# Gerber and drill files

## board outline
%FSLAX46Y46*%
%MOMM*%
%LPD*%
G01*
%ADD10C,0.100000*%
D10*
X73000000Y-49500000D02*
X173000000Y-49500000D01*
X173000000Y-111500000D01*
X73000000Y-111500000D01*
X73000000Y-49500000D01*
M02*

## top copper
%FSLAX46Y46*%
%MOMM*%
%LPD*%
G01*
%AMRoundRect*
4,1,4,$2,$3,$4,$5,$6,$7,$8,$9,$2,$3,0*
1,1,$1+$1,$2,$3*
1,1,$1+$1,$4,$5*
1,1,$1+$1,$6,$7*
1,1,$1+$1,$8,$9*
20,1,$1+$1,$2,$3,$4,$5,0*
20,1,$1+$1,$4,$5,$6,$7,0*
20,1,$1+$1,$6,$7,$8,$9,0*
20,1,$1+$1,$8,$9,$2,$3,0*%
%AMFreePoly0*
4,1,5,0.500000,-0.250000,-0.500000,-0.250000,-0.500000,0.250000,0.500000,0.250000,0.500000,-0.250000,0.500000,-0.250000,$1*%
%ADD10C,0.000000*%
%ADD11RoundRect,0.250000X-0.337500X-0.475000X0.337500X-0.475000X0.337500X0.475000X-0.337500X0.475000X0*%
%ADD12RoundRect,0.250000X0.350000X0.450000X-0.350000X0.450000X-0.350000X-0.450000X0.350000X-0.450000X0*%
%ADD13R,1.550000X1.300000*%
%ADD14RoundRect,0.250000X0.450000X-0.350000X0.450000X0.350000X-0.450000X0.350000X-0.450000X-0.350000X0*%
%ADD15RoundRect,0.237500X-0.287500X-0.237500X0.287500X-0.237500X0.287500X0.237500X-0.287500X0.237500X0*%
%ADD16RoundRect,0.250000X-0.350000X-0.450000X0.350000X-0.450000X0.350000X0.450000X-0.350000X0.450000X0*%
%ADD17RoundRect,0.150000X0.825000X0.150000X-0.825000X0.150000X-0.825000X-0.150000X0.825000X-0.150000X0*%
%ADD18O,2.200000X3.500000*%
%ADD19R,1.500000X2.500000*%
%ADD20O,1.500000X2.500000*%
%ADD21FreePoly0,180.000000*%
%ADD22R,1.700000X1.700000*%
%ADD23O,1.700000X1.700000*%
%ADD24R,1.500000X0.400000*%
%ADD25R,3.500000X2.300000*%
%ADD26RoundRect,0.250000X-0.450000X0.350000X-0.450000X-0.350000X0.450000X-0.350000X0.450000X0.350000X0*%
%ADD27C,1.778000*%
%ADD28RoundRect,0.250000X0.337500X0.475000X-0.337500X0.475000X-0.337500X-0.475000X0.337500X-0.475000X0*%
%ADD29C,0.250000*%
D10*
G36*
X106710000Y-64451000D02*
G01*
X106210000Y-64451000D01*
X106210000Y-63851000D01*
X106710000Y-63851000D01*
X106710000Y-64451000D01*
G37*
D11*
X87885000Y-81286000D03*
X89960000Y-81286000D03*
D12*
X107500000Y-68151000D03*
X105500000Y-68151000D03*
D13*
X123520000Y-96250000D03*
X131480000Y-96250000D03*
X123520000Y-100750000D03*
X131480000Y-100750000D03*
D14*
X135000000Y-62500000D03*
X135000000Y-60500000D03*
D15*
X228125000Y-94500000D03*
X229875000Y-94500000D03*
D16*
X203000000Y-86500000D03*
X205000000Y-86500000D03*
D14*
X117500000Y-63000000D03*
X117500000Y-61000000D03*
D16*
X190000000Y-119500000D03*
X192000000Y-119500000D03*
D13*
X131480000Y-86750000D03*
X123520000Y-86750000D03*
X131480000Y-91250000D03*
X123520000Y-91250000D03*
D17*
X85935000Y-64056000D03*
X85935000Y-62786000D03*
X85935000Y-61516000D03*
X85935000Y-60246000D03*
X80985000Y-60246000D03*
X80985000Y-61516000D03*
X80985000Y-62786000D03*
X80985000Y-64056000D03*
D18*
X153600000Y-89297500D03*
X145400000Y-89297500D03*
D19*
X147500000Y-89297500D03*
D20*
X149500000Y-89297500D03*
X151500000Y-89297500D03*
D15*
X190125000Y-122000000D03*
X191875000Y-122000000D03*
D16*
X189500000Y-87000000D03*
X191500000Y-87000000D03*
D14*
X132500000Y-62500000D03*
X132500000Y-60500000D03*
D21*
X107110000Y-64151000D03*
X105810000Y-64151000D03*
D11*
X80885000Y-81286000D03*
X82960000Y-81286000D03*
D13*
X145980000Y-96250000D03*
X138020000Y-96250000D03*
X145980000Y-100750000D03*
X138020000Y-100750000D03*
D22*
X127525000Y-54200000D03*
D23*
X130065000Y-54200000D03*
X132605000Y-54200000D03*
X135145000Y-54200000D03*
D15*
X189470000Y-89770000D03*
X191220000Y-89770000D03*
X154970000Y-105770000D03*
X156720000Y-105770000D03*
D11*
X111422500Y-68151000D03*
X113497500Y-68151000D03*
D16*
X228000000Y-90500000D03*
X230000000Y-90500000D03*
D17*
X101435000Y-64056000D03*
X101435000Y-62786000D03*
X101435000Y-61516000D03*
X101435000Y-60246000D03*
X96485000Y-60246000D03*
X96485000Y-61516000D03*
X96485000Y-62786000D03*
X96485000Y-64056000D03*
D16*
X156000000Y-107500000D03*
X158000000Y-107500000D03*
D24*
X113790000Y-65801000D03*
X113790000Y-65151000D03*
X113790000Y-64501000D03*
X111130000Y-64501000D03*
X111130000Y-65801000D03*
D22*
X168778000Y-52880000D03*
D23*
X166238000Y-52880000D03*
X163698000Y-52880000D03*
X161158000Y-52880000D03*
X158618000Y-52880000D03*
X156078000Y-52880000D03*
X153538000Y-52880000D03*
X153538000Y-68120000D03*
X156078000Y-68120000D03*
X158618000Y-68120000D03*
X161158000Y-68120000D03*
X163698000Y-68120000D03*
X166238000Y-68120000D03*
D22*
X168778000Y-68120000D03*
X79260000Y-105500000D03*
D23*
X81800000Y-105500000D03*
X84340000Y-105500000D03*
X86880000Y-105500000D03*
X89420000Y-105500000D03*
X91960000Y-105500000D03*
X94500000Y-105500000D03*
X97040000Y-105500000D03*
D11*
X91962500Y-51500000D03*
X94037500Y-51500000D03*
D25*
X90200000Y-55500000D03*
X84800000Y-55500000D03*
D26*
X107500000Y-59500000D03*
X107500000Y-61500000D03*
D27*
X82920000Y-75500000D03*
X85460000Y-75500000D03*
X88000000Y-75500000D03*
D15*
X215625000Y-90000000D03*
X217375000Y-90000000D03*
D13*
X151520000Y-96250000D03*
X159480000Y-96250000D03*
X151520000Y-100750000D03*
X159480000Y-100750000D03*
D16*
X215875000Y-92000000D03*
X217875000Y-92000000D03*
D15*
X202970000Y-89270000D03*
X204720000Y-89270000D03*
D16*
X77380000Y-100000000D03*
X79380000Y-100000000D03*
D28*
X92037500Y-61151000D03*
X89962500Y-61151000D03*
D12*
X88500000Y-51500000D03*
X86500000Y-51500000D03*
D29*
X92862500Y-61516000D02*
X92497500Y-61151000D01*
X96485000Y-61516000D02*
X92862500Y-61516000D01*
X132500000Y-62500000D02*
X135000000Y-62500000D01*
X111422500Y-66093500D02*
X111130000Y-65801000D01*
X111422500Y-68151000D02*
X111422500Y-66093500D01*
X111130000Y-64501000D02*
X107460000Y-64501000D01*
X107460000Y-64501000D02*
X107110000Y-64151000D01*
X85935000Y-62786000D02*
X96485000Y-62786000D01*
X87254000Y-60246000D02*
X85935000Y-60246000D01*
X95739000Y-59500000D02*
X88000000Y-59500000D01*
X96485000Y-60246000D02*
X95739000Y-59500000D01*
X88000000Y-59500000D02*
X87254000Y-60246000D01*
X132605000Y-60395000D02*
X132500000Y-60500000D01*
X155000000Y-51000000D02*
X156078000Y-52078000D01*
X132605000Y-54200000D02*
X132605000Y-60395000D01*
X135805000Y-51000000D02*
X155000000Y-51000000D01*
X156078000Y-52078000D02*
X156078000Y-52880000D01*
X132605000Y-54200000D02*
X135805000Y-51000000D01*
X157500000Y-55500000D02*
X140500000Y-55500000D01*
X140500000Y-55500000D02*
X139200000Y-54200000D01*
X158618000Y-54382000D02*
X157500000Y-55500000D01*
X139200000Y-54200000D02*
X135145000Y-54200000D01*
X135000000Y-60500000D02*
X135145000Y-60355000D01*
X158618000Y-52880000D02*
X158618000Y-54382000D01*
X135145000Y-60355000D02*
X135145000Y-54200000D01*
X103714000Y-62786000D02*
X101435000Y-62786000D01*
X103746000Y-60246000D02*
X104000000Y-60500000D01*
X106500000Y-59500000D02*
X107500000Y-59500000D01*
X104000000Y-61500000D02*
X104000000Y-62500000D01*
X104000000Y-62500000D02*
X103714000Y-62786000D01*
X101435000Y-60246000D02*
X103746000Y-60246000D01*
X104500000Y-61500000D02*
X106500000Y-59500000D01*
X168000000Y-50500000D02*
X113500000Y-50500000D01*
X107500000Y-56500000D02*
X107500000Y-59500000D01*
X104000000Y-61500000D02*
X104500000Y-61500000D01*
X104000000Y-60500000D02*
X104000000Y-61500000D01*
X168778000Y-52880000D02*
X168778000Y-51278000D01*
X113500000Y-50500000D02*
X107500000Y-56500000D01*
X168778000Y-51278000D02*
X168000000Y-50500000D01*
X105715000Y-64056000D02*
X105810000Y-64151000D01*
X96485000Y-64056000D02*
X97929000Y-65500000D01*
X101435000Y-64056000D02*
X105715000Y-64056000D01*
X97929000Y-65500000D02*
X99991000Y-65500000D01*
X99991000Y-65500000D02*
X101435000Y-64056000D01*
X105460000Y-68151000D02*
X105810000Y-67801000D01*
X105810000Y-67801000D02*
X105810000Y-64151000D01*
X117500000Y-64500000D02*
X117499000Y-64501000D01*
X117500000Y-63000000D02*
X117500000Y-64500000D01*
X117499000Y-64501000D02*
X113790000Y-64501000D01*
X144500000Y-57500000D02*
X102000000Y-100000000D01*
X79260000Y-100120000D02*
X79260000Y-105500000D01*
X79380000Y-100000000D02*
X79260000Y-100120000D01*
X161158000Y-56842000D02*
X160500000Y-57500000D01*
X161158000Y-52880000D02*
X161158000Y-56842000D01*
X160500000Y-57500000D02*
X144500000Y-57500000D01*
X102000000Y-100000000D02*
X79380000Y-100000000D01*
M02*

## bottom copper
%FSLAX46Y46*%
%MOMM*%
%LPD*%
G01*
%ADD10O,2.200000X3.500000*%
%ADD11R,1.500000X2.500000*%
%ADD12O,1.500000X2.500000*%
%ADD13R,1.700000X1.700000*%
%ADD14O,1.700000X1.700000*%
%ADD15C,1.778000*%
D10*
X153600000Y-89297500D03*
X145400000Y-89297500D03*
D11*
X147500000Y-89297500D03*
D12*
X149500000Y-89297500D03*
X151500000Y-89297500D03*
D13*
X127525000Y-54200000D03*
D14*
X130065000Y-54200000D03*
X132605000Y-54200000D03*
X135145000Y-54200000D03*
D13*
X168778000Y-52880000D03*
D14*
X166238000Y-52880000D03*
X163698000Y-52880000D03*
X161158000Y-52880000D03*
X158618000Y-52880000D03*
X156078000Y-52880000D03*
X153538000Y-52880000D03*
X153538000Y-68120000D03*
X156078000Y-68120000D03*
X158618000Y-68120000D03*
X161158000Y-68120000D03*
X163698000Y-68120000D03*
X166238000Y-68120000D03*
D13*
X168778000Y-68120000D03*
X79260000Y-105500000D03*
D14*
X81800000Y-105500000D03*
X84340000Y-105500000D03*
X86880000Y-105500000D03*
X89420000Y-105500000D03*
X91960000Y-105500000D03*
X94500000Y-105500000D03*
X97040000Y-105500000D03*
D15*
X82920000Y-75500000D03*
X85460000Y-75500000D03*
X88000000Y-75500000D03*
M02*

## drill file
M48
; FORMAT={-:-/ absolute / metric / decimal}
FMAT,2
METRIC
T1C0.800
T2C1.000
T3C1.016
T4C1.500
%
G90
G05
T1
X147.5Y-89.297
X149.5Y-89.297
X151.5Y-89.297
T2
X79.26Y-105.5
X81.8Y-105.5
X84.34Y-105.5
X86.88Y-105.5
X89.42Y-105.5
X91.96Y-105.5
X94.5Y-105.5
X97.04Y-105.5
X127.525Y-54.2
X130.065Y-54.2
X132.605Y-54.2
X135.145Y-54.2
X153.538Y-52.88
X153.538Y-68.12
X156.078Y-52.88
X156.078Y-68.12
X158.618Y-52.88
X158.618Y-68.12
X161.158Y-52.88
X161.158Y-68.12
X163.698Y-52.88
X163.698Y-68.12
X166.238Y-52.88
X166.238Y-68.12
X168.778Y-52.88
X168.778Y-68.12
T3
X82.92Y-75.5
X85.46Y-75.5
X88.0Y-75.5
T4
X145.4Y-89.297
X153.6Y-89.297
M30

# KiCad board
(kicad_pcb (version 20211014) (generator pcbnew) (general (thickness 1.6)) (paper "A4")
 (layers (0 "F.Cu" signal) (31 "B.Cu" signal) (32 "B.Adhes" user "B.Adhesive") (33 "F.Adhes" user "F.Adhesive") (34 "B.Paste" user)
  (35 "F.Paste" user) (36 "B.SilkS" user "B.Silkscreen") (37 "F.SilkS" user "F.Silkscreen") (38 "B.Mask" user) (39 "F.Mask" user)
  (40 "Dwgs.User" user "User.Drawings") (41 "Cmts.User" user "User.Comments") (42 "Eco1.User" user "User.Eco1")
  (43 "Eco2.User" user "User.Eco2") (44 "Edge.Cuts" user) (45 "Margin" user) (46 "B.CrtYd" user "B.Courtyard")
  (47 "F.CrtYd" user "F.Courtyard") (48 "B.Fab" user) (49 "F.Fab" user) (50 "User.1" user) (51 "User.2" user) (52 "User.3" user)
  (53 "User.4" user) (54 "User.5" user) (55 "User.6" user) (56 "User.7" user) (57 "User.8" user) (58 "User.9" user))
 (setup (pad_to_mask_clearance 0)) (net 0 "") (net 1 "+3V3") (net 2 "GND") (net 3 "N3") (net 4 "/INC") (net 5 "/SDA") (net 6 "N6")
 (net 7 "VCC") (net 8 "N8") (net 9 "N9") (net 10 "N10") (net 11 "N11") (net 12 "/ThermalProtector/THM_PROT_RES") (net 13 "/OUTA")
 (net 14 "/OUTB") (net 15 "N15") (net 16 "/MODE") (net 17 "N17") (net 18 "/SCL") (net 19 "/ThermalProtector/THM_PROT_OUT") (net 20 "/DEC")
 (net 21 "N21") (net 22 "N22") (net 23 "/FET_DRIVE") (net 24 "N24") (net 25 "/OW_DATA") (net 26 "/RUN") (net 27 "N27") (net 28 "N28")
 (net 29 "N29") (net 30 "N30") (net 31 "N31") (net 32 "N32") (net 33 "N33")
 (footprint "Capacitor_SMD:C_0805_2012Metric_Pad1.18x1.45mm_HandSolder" (layer "F.Cu") (at 88.9225 81.286)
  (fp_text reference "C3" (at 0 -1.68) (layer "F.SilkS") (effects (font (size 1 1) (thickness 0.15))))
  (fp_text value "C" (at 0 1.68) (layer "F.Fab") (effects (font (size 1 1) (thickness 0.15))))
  (pad "1" smd roundrect (at -1.0375 0) (size 1.175 1.45) (layers "F.Cu" "F.Paste" "F.Mask") (roundrect_rratio 0.212766) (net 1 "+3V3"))
  (pad "2" smd roundrect (at 1.0375 0) (size 1.175 1.45) (layers "F.Cu" "F.Paste" "F.Mask") (roundrect_rratio 0.212766) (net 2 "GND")))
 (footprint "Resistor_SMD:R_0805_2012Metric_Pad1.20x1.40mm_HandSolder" (layer "F.Cu") (at 106.5 68.151 180)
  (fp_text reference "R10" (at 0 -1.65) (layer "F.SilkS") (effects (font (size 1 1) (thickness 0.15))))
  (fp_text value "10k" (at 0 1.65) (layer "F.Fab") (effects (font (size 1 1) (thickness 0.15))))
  (pad "1" smd roundrect (at -1 0 180) (size 1.2 1.4) (layers "F.Cu" "F.Paste" "F.Mask") (roundrect_rratio 0.208333) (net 1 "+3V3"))
  (pad "2" smd roundrect (at 1 0 180) (size 1.2 1.4) (layers "F.Cu" "F.Paste" "F.Mask") (roundrect_rratio 0.208333) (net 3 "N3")))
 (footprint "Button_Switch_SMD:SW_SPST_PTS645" (layer "F.Cu") (at 127.5 98.5)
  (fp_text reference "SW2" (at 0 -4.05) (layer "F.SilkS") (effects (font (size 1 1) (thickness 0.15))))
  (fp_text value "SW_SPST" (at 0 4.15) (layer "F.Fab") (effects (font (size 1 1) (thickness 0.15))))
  (pad "1" smd rect (at -3.98 -2.25) (size 1.55 1.3) (layers "F.Cu" "F.Paste" "F.Mask") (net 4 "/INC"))
  (pad "1" smd rect (at 3.98 -2.25) (size 1.55 1.3) (layers "F.Cu" "F.Paste" "F.Mask") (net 4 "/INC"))
  (pad "2" smd rect (at -3.98 2.25) (size 1.55 1.3) (layers "F.Cu" "F.Paste" "F.Mask") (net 2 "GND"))
  (pad "2" smd rect (at 3.98 2.25) (size 1.55 1.3) (layers "F.Cu" "F.Paste" "F.Mask") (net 2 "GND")))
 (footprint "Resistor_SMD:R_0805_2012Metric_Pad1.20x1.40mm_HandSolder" (layer "F.Cu") (at 135 61.5 90)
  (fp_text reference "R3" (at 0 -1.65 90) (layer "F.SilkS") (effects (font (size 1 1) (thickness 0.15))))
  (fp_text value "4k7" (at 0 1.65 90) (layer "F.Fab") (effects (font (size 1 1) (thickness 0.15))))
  (pad "1" smd roundrect (at -1 0 90) (size 1.2 1.4) (layers "F.Cu" "F.Paste" "F.Mask") (roundrect_rratio 0.208333) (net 1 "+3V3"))
  (pad "2" smd roundrect (at 1 0 90) (size 1.2 1.4) (layers "F.Cu" "F.Paste" "F.Mask") (roundrect_rratio 0.208333) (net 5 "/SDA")))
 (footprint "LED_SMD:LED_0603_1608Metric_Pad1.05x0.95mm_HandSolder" (layer "F.Cu") (at 229 94.5)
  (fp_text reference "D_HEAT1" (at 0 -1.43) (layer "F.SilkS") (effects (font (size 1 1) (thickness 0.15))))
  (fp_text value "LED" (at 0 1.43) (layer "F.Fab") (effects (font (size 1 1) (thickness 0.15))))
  (pad "1" smd roundrect (at -0.875 0) (size 1.05 0.95) (layers "F.Cu" "F.Paste" "F.Mask") (roundrect_rratio 0.25) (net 2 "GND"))
  (pad "2" smd roundrect (at 0.875 0) (size 1.05 0.95) (layers "F.Cu" "F.Paste" "F.Mask") (roundrect_rratio 0.25) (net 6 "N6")))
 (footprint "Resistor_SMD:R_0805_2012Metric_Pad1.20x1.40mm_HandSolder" (layer "F.Cu") (at 204 86.5)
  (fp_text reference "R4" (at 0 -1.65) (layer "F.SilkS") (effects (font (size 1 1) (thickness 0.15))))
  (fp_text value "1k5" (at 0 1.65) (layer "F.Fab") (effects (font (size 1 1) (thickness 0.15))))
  (pad "1" smd roundrect (at -1 0) (size 1.2 1.4) (layers "F.Cu" "F.Paste" "F.Mask") (roundrect_rratio 0.208333) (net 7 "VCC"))
  (pad "2" smd roundrect (at 1 0) (size 1.2 1.4) (layers "F.Cu" "F.Paste" "F.Mask") (roundrect_rratio 0.208333) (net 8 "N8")))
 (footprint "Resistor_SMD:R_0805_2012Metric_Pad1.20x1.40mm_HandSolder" (layer "F.Cu") (at 117.5 62 90)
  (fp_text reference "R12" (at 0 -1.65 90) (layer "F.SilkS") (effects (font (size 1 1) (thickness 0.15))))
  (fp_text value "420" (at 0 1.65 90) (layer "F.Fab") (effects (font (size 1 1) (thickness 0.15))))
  (pad "1" smd roundrect (at -1 0 90) (size 1.2 1.4) (layers "F.Cu" "F.Paste" "F.Mask") (roundrect_rratio 0.208333) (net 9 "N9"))
  (pad "2" smd roundrect (at 1 0 90) (size 1.2 1.4) (layers "F.Cu" "F.Paste" "F.Mask") (roundrect_rratio 0.208333) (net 2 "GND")))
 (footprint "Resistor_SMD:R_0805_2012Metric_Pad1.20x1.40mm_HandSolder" (layer "F.Cu") (at 191 119.5)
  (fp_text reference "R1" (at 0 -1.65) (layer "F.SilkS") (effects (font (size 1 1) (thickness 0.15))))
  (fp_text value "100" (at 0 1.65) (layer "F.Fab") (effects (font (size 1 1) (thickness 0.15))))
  (pad "1" smd roundrect (at -1 0) (size 1.2 1.4) (layers "F.Cu" "F.Paste" "F.Mask") (roundrect_rratio 0.208333) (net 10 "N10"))
  (pad "2" smd roundrect (at 1 0) (size 1.2 1.4) (layers "F.Cu" "F.Paste" "F.Mask") (roundrect_rratio 0.208333) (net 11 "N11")))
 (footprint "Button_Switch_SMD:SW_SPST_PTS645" (layer "F.Cu") (at 127.5 89)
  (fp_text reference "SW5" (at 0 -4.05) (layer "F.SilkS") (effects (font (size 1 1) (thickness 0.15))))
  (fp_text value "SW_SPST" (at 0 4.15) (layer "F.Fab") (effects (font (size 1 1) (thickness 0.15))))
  (pad "1" smd rect (at 3.98 -2.25) (size 1.55 1.3) (layers "F.Cu" "F.Paste" "F.Mask") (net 2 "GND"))
  (pad "1" smd rect (at -3.98 -2.25) (size 1.55 1.3) (layers "F.Cu" "F.Paste" "F.Mask") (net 2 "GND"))
  (pad "2" smd rect (at 3.98 2.25) (size 1.55 1.3) (layers "F.Cu" "F.Paste" "F.Mask") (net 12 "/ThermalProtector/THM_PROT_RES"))
  (pad "2" smd rect (at -3.98 2.25) (size 1.55 1.3) (layers "F.Cu" "F.Paste" "F.Mask") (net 12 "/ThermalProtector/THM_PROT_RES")))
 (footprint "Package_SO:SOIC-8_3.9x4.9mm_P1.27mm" (layer "F.Cu") (at 83.46 62.151 180)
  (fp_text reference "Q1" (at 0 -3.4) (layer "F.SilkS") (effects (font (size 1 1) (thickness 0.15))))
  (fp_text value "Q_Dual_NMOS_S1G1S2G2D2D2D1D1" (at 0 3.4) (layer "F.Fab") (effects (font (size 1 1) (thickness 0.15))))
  (pad "1" smd roundrect (at -2.475 -1.905 180) (size 1.95 0.6) (layers "F.Cu" "F.Paste" "F.Mask") (roundrect_rratio 0.25) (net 2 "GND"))
  (pad "2" smd roundrect (at -2.475 -0.635 180) (size 1.95 0.6) (layers "F.Cu" "F.Paste" "F.Mask") (roundrect_rratio 0.25) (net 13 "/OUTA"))
  (pad "3" smd roundrect (at -2.475 0.635 180) (size 1.95 0.6) (layers "F.Cu" "F.Paste" "F.Mask") (roundrect_rratio 0.25) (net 2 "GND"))
  (pad "4" smd roundrect (at -2.475 1.905 180) (size 1.95 0.6) (layers "F.Cu" "F.Paste" "F.Mask") (roundrect_rratio 0.25) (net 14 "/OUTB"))
  (pad "5" smd roundrect (at 2.475 1.905 180) (size 1.95 0.6) (layers "F.Cu" "F.Paste" "F.Mask") (roundrect_rratio 0.25) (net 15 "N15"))
  (pad "6" smd roundrect (at 2.475 0.635 180) (size 1.95 0.6) (layers "F.Cu" "F.Paste" "F.Mask") (roundrect_rratio 0.25) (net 15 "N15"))
  (pad "7" smd roundrect (at 2.475 -0.635 180) (size 1.95 0.6) (layers "F.Cu" "F.Paste" "F.Mask") (roundrect_rratio 0.25) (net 15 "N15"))
  (pad "8" smd roundrect (at 2.475 -1.905 180) (size 1.95 0.6) (layers "F.Cu" "F.Paste" "F.Mask") (roundrect_rratio 0.25) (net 15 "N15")))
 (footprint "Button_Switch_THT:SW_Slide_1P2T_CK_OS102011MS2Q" (layer "F.Cu") (at 147.5 89.2975)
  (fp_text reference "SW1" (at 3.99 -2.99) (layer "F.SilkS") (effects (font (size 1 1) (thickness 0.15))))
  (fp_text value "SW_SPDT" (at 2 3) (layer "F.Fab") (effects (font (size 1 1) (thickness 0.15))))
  (pad "" thru_hole oval (at 6.1 0) (size 2.2 3.5) (drill 1.5) (layers *.Cu *.Mask))
  (pad "" thru_hole oval (at -2.1 0) (size 2.2 3.5) (drill 1.5) (layers *.Cu *.Mask))
  (pad "1" thru_hole rect (at 0 0) (size 1.5 2.5) (drill 0.8) (layers *.Cu *.Mask) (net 1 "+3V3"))
  (pad "2" thru_hole oval (at 2 0) (size 1.5 2.5) (drill 0.8) (layers *.Cu *.Mask) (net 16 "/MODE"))
  (pad "3" thru_hole oval (at 4 0) (size 1.5 2.5) (drill 0.8) (layers *.Cu *.Mask) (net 2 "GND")))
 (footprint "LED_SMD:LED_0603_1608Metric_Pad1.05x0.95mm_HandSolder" (layer "F.Cu") (at 191 122)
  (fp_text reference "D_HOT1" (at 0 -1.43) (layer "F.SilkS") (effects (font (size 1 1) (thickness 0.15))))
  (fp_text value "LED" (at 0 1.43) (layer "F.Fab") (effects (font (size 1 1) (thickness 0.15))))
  (pad "1" smd roundrect (at -0.875 0) (size 1.05 0.95) (layers "F.Cu" "F.Paste" "F.Mask") (roundrect_rratio 0.25) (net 2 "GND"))
  (pad "2" smd roundrect (at 0.875 0) (size 1.05 0.95) (layers "F.Cu" "F.Paste" "F.Mask") (roundrect_rratio 0.25) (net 11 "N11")))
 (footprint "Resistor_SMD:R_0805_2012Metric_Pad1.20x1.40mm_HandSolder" (layer "F.Cu") (at 190.5 87)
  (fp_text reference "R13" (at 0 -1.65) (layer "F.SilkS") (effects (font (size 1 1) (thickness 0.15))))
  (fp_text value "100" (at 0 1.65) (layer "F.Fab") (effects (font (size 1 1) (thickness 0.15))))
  (pad "1" smd roundrect (at -1 0) (size 1.2 1.4) (layers "F.Cu" "F.Paste" "F.Mask") (roundrect_rratio 0.208333) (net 1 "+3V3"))
  (pad "2" smd roundrect (at 1 0) (size 1.2 1.4) (layers "F.Cu" "F.Paste" "F.Mask") (roundrect_rratio 0.208333) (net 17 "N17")))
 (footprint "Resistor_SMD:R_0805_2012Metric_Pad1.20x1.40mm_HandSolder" (layer "F.Cu") (at 132.5 61.5 90)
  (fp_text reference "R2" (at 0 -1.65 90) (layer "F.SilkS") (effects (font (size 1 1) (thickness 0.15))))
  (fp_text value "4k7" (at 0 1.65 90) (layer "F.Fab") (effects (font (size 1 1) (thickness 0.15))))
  (pad "1" smd roundrect (at -1 0 90) (size 1.2 1.4) (layers "F.Cu" "F.Paste" "F.Mask") (roundrect_rratio 0.208333) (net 1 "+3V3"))
  (pad "2" smd roundrect (at 1 0 90) (size 1.2 1.4) (layers "F.Cu" "F.Paste" "F.Mask") (roundrect_rratio 0.208333) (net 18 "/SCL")))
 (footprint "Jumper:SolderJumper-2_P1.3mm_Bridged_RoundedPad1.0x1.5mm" (layer "F.Cu") (at 106.46 64.151 180)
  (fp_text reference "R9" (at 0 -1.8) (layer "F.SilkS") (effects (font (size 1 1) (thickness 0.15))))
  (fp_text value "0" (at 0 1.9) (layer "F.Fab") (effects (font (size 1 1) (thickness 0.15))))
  (fp_poly (pts (xy 0.25 -0.3) (xy -0.25 -0.3) (xy -0.25 0.3) (xy 0.25 0.3)) (layer "F.Cu") (width 0) (fill solid))
  (pad "1" smd custom (at -0.65 0 180) (size 1 0.5) (layers "F.Cu" "F.Mask") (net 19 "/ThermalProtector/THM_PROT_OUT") (zone_connect 2)
   (options (clearance outline) (anchor rect)) (primitives))
  (pad "2" smd custom (at 0.65 0 180) (size 1 0.5) (layers "F.Cu" "F.Mask") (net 3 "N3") (zone_connect 2)
   (options (clearance outline) (anchor rect)) (primitives)))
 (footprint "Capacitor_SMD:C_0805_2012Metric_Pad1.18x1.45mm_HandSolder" (layer "F.Cu") (at 81.9225 81.286)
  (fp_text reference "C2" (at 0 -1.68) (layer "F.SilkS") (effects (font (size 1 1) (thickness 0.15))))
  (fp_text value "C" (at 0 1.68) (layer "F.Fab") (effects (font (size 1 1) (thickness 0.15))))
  (pad "1" smd roundrect (at -1.0375 0) (size 1.175 1.45) (layers "F.Cu" "F.Paste" "F.Mask") (roundrect_rratio 0.212766) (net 7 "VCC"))
  (pad "2" smd roundrect (at 1.0375 0) (size 1.175 1.45) (layers "F.Cu" "F.Paste" "F.Mask") (roundrect_rratio 0.212766) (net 2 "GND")))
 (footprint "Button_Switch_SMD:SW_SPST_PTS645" (layer "F.Cu") (at 142 98.5)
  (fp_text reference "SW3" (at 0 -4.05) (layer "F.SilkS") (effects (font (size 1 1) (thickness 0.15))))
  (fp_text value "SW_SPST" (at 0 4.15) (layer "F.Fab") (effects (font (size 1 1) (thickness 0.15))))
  (pad "1" smd rect (at 3.98 -2.25) (size 1.55 1.3) (layers "F.Cu" "F.Paste" "F.Mask") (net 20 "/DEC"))
  (pad "1" smd rect (at -3.98 -2.25) (size 1.55 1.3) (layers "F.Cu" "F.Paste" "F.Mask") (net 20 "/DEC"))
  (pad "2" smd rect (at 3.98 2.25) (size 1.55 1.3) (layers "F.Cu" "F.Paste" "F.Mask") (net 2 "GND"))
  (pad "2" smd rect (at -3.98 2.25) (size 1.55 1.3) (layers "F.Cu" "F.Paste" "F.Mask") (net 2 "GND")))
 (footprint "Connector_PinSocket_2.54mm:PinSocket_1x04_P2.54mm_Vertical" (layer "F.Cu") (at 127.525 54.2 90)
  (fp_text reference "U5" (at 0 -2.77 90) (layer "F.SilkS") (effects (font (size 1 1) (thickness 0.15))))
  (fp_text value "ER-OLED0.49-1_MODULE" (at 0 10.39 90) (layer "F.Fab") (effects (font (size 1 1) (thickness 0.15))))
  (pad "1" thru_hole rect (at 0 0 90) (size 1.7 1.7) (drill 1) (layers *.Cu *.Mask) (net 2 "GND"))
  (pad "2" thru_hole oval (at 0 2.54 90) (size 1.7 1.7) (drill 1) (layers *.Cu *.Mask) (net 1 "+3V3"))
  (pad "3" thru_hole oval (at 0 5.08 90) (size 1.7 1.7) (drill 1) (layers *.Cu *.Mask) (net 18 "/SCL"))
  (pad "4" thru_hole oval (at 0 7.62 90) (size 1.7 1.7) (drill 1) (layers *.Cu *.Mask) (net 5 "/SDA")))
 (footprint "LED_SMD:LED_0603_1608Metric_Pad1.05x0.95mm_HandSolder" (layer "F.Cu") (at 190.345 89.77)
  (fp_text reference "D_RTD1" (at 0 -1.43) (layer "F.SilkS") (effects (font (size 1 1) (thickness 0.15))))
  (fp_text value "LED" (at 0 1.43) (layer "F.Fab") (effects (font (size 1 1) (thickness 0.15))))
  (pad "1" smd roundrect (at -0.875 0) (size 1.05 0.95) (layers "F.Cu" "F.Paste" "F.Mask") (roundrect_rratio 0.25)
   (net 19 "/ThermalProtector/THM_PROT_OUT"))
  (pad "2" smd roundrect (at 0.875 0) (size 1.05 0.95) (layers "F.Cu" "F.Paste" "F.Mask") (roundrect_rratio 0.25) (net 17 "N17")))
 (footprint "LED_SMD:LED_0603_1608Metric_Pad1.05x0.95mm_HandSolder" (layer "F.Cu") (at 155.845 105.77)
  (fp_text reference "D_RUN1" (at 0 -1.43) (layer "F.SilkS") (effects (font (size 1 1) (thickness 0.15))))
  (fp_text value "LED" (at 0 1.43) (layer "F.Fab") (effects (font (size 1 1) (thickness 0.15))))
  (pad "1" smd roundrect (at -0.875 0) (size 1.05 0.95) (layers "F.Cu" "F.Paste" "F.Mask") (roundrect_rratio 0.25) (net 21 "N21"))
  (pad "2" smd roundrect (at 0.875 0) (size 1.05 0.95) (layers "F.Cu" "F.Paste" "F.Mask") (roundrect_rratio 0.25) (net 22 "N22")))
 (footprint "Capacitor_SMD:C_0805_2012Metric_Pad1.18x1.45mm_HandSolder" (layer "F.Cu") (at 112.46 68.151)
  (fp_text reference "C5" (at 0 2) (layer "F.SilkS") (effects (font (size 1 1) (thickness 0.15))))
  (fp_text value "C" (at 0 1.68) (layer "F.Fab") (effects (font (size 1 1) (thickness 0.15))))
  (pad "1" smd roundrect (at -1.0375 0) (size 1.175 1.45) (layers "F.Cu" "F.Paste" "F.Mask") (roundrect_rratio 0.212766) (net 1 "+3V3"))
  (pad "2" smd roundrect (at 1.0375 0) (size 1.175 1.45) (layers "F.Cu" "F.Paste" "F.Mask") (roundrect_rratio 0.212766) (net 2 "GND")))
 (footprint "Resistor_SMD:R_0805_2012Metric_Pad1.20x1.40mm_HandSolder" (layer "F.Cu") (at 229 90.5)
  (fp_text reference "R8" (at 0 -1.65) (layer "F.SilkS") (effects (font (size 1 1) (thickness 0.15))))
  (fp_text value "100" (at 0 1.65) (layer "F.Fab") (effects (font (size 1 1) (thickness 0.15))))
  (pad "1" smd roundrect (at -1 0) (size 1.2 1.4) (layers "F.Cu" "F.Paste" "F.Mask") (roundrect_rratio 0.208333) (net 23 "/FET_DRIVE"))
  (pad "2" smd roundrect (at 1 0) (size 1.2 1.4) (layers "F.Cu" "F.Paste" "F.Mask") (roundrect_rratio 0.208333) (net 6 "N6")))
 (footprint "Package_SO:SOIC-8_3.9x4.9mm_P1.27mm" (layer "F.Cu") (at 98.96 62.151 180)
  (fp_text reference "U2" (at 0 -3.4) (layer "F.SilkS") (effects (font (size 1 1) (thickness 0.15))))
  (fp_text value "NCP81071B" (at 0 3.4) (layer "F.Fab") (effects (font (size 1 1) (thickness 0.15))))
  (pad "1" smd roundrect (at -2.475 -1.905 180) (size 1.95 0.6) (layers "F.Cu" "F.Paste" "F.Mask") (roundrect_rratio 0.25) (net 3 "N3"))
  (pad "2" smd roundrect (at -2.475 -0.635 180) (size 1.95 0.6) (layers "F.Cu" "F.Paste" "F.Mask") (roundrect_rratio 0.25)
   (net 23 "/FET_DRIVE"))
  (pad "3" smd roundrect (at -2.475 0.635 180) (size 1.95 0.6) (layers "F.Cu" "F.Paste" "F.Mask") (roundrect_rratio 0.25) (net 2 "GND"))
  (pad "4" smd roundrect (at -2.475 1.905 180) (size 1.95 0.6) (layers "F.Cu" "F.Paste" "F.Mask") (roundrect_rratio 0.25)
   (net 23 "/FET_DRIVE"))
  (pad "5" smd roundrect (at 2.475 1.905 180) (size 1.95 0.6) (layers "F.Cu" "F.Paste" "F.Mask") (roundrect_rratio 0.25) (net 14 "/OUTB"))
  (pad "6" smd roundrect (at 2.475 0.635 180) (size 1.95 0.6) (layers "F.Cu" "F.Paste" "F.Mask") (roundrect_rratio 0.25) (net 7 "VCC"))
  (pad "7" smd roundrect (at 2.475 -0.635 180) (size 1.95 0.6) (layers "F.Cu" "F.Paste" "F.Mask") (roundrect_rratio 0.25) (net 13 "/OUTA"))
  (pad "8" smd roundrect (at 2.475 -1.905 180) (size 1.95 0.6) (layers "F.Cu" "F.Paste" "F.Mask") (roundrect_rratio 0.25) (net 3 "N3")))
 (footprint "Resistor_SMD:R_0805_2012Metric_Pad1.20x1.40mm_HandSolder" (layer "F.Cu") (at 157 107.5)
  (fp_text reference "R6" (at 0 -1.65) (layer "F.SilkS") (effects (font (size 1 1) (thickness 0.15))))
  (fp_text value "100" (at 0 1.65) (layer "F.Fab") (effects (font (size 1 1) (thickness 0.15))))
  (pad "1" smd roundrect (at -1 0) (size 1.2 1.4) (layers "F.Cu" "F.Paste" "F.Mask") (roundrect_rratio 0.208333) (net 21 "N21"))
  (pad "2" smd roundrect (at 1 0) (size 1.2 1.4) (layers "F.Cu" "F.Paste" "F.Mask") (roundrect_rratio 0.208333) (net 2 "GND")))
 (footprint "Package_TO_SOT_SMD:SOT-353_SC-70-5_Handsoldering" (layer "F.Cu") (at 112.46 65.151 180)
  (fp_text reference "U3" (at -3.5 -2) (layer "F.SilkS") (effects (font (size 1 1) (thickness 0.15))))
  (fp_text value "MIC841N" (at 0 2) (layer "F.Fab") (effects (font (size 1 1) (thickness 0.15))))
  (pad "1" smd rect (at -1.33 -0.65 180) (size 1.5 0.4) (layers "F.Cu" "F.Paste" "F.Mask") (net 12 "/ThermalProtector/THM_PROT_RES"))
  (pad "2" smd rect (at -1.33 0 180) (size 1.5 0.4) (layers "F.Cu" "F.Paste" "F.Mask") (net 2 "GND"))
  (pad "3" smd rect (at -1.33 0.65 180) (size 1.5 0.4) (layers "F.Cu" "F.Paste" "F.Mask") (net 9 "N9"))
  (pad "4" smd rect (at 1.33 0.65 180) (size 1.5 0.4) (layers "F.Cu" "F.Paste" "F.Mask") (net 19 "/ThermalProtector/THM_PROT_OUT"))
  (pad "5" smd rect (at 1.33 -0.65 180) (size 1.5 0.4) (layers "F.Cu" "F.Paste" "F.Mask") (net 1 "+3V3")))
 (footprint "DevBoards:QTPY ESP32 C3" (layer "F.Cu") (at 167 60.5 -90)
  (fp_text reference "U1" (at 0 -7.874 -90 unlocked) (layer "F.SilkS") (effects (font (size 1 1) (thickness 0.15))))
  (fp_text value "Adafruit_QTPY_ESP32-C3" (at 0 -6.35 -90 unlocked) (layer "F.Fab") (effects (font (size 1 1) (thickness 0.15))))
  (pad "1" thru_hole rect (at -7.62 -1.778 270) (size 1.7 1.7) (drill 1) (layers *.Cu *.Mask) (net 23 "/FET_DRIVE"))
  (pad "2" thru_hole oval (at -7.62 0.762 270) (size 1.7 1.7) (drill 1) (layers *.Cu *.Mask) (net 10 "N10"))
  (pad "3" thru_hole oval (at -7.62 3.302 270) (size 1.7 1.7) (drill 1) (layers *.Cu *.Mask) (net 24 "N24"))
  (pad "4" thru_hole oval (at -7.62 5.842 270) (size 1.7 1.7) (drill 1) (layers *.Cu *.Mask) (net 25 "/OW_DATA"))
  (pad "5" thru_hole oval (at -7.62 8.382 270) (size 1.7 1.7) (drill 1) (layers *.Cu *.Mask) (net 5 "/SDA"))
  (pad "6" thru_hole oval (at -7.62 10.922 270) (size 1.7 1.7) (drill 1) (layers *.Cu *.Mask) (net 18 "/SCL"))
  (pad "7" thru_hole oval (at -7.62 13.462 270) (size 1.7 1.7) (drill 1) (layers *.Cu *.Mask) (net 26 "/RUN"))
  (pad "8" thru_hole oval (at 7.62 13.462 270) (size 1.7 1.7) (drill 1) (layers *.Cu *.Mask) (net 20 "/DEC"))
  (pad "9" thru_hole oval (at 7.62 10.922 270) (size 1.7 1.7) (drill 1) (layers *.Cu *.Mask) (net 4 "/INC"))
  (pad "10" thru_hole oval (at 7.62 8.382 270) (size 1.7 1.7) (drill 1) (layers *.Cu *.Mask) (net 16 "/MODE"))
  (pad "11" thru_hole oval (at 7.62 5.842 270) (size 1.7 1.7) (drill 1) (layers *.Cu *.Mask) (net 22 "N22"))
  (pad "12" thru_hole oval (at 7.62 3.302 270) (size 1.7 1.7) (drill 1) (layers *.Cu *.Mask) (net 1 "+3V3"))
  (pad "13" thru_hole oval (at 7.62 0.762 270) (size 1.7 1.7) (drill 1) (layers *.Cu *.Mask) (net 2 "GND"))
  (pad "14" thru_hole rect (at 7.62 -1.778 270) (size 1.7 1.7) (drill 1) (layers *.Cu *.Mask) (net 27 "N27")))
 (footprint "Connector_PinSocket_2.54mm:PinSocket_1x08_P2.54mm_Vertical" (layer "F.Cu") (at 79.26 105.5 90)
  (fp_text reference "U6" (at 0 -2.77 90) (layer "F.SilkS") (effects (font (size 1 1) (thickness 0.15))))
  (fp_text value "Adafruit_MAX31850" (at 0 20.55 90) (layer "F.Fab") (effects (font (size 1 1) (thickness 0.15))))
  (pad "1" thru_hole rect (at 0 0 90) (size 1.7 1.7) (drill 1) (layers *.Cu *.Mask) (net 25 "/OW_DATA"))
  (pad "2" thru_hole oval (at 0 2.54 90) (size 1.7 1.7) (drill 1) (layers *.Cu *.Mask) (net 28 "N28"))
  (pad "3" thru_hole oval (at 0 5.08 90) (size 1.7 1.7) (drill 1) (layers *.Cu *.Mask) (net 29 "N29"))
  (pad "4" thru_hole oval (at 0 7.62 90) (size 1.7 1.7) (drill 1) (layers *.Cu *.Mask) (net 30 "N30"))
  (pad "5" thru_hole oval (at 0 10.16 90) (size 1.7 1.7) (drill 1) (layers *.Cu *.Mask) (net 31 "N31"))
  (pad "6" thru_hole oval (at 0 12.7 90) (size 1.7 1.7) (drill 1) (layers *.Cu *.Mask) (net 1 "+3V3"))
  (pad "7" thru_hole oval (at 0 15.24 90) (size 1.7 1.7) (drill 1) (layers *.Cu *.Mask) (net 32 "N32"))
  (pad "8" thru_hole oval (at 0 17.78 90) (size 1.7 1.7) (drill 1) (layers *.Cu *.Mask) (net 2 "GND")))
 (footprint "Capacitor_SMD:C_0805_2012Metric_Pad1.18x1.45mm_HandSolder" (layer "F.Cu") (at 93 51.5)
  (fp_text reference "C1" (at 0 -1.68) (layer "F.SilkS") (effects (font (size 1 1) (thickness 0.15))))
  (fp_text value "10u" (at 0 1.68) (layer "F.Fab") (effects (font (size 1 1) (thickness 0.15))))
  (pad "1" smd roundrect (at -1.0375 0) (size 1.175 1.45) (layers "F.Cu" "F.Paste" "F.Mask") (roundrect_rratio 0.212766) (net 7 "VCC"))
  (pad "2" smd roundrect (at 1.0375 0) (size 1.175 1.45) (layers "F.Cu" "F.Paste" "F.Mask") (roundrect_rratio 0.212766) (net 2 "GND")))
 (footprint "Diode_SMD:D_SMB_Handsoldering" (layer "F.Cu") (at 87.5 55.5 180)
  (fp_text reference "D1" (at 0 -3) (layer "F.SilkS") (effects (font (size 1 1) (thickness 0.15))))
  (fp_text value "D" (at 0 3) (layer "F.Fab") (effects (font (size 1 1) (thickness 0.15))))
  (pad "1" smd rect (at -2.7 0 180) (size 3.5 2.3) (layers "F.Cu" "F.Paste" "F.Mask") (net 7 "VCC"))
  (pad "2" smd rect (at 2.7 0 180) (size 3.5 2.3) (layers "F.Cu" "F.Paste" "F.Mask") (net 15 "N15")))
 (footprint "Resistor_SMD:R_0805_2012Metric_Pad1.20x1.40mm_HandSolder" (layer "F.Cu") (at 107.5 60.5 -90)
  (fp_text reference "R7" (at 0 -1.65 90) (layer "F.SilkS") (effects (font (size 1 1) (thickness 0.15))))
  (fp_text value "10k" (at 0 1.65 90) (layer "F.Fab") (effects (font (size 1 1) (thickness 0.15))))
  (pad "1" smd roundrect (at -1 0 270) (size 1.2 1.4) (layers "F.Cu" "F.Paste" "F.Mask") (roundrect_rratio 0.208333) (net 23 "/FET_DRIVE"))
  (pad "2" smd roundrect (at 1 0 270) (size 1.2 1.4) (layers "F.Cu" "F.Paste" "F.Mask") (roundrect_rratio 0.208333) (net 2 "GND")))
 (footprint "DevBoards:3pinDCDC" (layer "F.Cu") (at 85.46 75.5)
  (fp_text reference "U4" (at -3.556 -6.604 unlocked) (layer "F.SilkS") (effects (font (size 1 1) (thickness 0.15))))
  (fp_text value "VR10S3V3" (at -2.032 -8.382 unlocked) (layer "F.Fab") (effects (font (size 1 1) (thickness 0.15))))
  (pad "1" thru_hole circle (at -2.54 0) (size 1.778 1.778) (drill 1.016) (layers *.Cu *.Mask) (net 7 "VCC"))
  (pad "2" thru_hole circle (at 0 0) (size 1.778 1.778) (drill 1.016) (layers *.Cu *.Mask) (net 2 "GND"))
  (pad "3" thru_hole circle (at 2.54 0) (size 1.778 1.778) (drill 1.016) (layers *.Cu *.Mask) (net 1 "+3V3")))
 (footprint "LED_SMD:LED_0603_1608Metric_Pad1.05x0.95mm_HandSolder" (layer "F.Cu") (at 216.5 90)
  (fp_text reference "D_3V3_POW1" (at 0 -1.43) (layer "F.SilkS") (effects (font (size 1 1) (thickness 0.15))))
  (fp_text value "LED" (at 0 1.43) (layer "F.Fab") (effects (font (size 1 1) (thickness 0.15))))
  (pad "1" smd roundrect (at -0.875 0) (size 1.05 0.95) (layers "F.Cu" "F.Paste" "F.Mask") (roundrect_rratio 0.25) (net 2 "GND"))
  (pad "2" smd roundrect (at 0.875 0) (size 1.05 0.95) (layers "F.Cu" "F.Paste" "F.Mask") (roundrect_rratio 0.25) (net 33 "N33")))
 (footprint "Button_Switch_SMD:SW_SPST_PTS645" (layer "F.Cu") (at 155.5 98.5)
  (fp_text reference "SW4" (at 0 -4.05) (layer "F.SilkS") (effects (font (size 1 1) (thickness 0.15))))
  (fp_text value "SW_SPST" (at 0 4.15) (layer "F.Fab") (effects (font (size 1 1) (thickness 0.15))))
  (pad "1" smd rect (at -3.98 -2.25) (size 1.55 1.3) (layers "F.Cu" "F.Paste" "F.Mask") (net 26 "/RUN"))
  (pad "1" smd rect (at 3.98 -2.25) (size 1.55 1.3) (layers "F.Cu" "F.Paste" "F.Mask") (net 26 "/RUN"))
  (pad "2" smd rect (at -3.98 2.25) (size 1.55 1.3) (layers "F.Cu" "F.Paste" "F.Mask") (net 2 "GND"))
  (pad "2" smd rect (at 3.98 2.25) (size 1.55 1.3) (layers "F.Cu" "F.Paste" "F.Mask") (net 2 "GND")))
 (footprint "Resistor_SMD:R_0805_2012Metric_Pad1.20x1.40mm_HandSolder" (layer "F.Cu") (at 216.875 92)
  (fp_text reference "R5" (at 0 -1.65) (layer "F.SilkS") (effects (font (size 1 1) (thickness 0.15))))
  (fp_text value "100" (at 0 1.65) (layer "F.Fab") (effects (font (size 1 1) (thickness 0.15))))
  (pad "1" smd roundrect (at -1 0) (size 1.2 1.4) (layers "F.Cu" "F.Paste" "F.Mask") (roundrect_rratio 0.208333) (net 1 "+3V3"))
  (pad "2" smd roundrect (at 1 0) (size 1.2 1.4) (layers "F.Cu" "F.Paste" "F.Mask") (roundrect_rratio 0.208333) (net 33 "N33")))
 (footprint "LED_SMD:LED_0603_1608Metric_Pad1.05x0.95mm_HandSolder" (layer "F.Cu") (at 203.845 89.27)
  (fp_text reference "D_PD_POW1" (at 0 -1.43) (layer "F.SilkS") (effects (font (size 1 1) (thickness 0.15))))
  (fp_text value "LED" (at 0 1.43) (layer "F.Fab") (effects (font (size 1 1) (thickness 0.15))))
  (pad "1" smd roundrect (at -0.875 0) (size 1.05 0.95) (layers "F.Cu" "F.Paste" "F.Mask") (roundrect_rratio 0.25) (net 2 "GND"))
  (pad "2" smd roundrect (at 0.875 0) (size 1.05 0.95) (layers "F.Cu" "F.Paste" "F.Mask") (roundrect_rratio 0.25) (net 8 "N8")))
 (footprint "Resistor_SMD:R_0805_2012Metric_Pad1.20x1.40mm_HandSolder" (layer "F.Cu") (at 78.38 100)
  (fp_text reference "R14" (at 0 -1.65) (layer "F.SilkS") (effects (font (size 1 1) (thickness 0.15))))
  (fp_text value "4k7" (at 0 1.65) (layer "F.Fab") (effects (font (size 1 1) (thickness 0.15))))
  (pad "1" smd roundrect (at -1 0) (size 1.2 1.4) (layers "F.Cu" "F.Paste" "F.Mask") (roundrect_rratio 0.208333) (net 1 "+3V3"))
  (pad "2" smd roundrect (at 1 0) (size 1.2 1.4) (layers "F.Cu" "F.Paste" "F.Mask") (roundrect_rratio 0.208333) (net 25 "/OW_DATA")))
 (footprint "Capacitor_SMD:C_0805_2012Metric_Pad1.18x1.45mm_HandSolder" (layer "F.Cu") (at 91 61.151 180)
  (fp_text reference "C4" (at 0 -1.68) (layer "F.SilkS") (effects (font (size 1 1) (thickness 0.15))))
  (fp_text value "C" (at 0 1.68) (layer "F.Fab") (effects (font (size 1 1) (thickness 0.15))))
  (pad "1" smd roundrect (at -1.0375 0 180) (size 1.175 1.45) (layers "F.Cu" "F.Paste" "F.Mask") (roundrect_rratio 0.212766) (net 7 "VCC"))
  (pad "2" smd roundrect (at 1.0375 0 180) (size 1.175 1.45) (layers "F.Cu" "F.Paste" "F.Mask") (roundrect_rratio 0.212766) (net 2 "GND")))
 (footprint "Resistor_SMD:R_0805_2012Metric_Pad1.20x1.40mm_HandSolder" (layer "F.Cu") (at 87.5 51.5 180)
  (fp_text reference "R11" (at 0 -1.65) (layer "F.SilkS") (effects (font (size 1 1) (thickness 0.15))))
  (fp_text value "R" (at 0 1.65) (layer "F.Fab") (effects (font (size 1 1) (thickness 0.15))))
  (pad "1" smd roundrect (at -1 0 180) (size 1.2 1.4) (layers "F.Cu" "F.Paste" "F.Mask") (roundrect_rratio 0.208333) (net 7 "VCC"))
  (pad "2" smd roundrect (at 1 0 180) (size 1.2 1.4) (layers "F.Cu" "F.Paste" "F.Mask") (roundrect_rratio 0.208333) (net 15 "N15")))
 (gr_rect (start 73 49.5) (end 173 111.5) (layer "Edge.Cuts") (width 0.1) (fill none))
 (segment (start 92.8625 61.516) (end 92.4975 61.151) (width 0.25) (layer "F.Cu") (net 7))
 (segment (start 96.485 61.516) (end 92.8625 61.516) (width 0.25) (layer "F.Cu") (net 7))
 (segment (start 132.5 62.5) (end 135 62.5) (width 0.25) (layer "F.Cu") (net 1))
 (segment (start 111.4225 66.0935) (end 111.13 65.801) (width 0.25) (layer "F.Cu") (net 1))
 (segment (start 111.4225 68.151) (end 111.4225 66.0935) (width 0.25) (layer "F.Cu") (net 1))
 (segment (start 111.13 64.501) (end 107.46 64.501) (width 0.25) (layer "F.Cu") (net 19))
 (segment (start 107.46 64.501) (end 107.11 64.151) (width 0.25) (layer "F.Cu") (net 19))
 (segment (start 85.935 62.786) (end 96.485 62.786) (width 0.25) (layer "F.Cu") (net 13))
 (segment (start 87.254 60.246) (end 85.935 60.246) (width 0.25) (layer "F.Cu") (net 14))
 (segment (start 95.739 59.5) (end 88 59.5) (width 0.25) (layer "F.Cu") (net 14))
 (segment (start 96.485 60.246) (end 95.739 59.5) (width 0.25) (layer "F.Cu") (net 14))
 (segment (start 88 59.5) (end 87.254 60.246) (width 0.25) (layer "F.Cu") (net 14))
 (segment (start 132.605 60.395) (end 132.5 60.5) (width 0.25) (layer "F.Cu") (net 18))
 (segment (start 155 51) (end 156.078 52.078) (width 0.25) (layer "F.Cu") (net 18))
 (segment (start 132.605 54.2) (end 132.605 60.395) (width 0.25) (layer "F.Cu") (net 18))
 (segment (start 135.805 51) (end 155 51) (width 0.25) (layer "F.Cu") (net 18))
 (segment (start 156.078 52.078) (end 156.078 52.88) (width 0.25) (layer "F.Cu") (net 18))
 (segment (start 132.605 54.2) (end 135.805 51) (width 0.25) (layer "F.Cu") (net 18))
 (segment (start 157.5 55.5) (end 140.5 55.5) (width 0.25) (layer "F.Cu") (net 5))
 (segment (start 140.5 55.5) (end 139.2 54.2) (width 0.25) (layer "F.Cu") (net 5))
 (segment (start 158.618 54.382) (end 157.5 55.5) (width 0.25) (layer "F.Cu") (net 5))
 (segment (start 139.2 54.2) (end 135.145 54.2) (width 0.25) (layer "F.Cu") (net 5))
 (segment (start 135 60.5) (end 135.145 60.355) (width 0.25) (layer "F.Cu") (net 5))
 (segment (start 158.618 52.88) (end 158.618 54.382) (width 0.25) (layer "F.Cu") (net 5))
 (segment (start 135.145 60.355) (end 135.145 54.2) (width 0.25) (layer "F.Cu") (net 5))
 (segment (start 103.714 62.786) (end 101.435 62.786) (width 0.25) (layer "F.Cu") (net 23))
 (segment (start 103.746 60.246) (end 104 60.5) (width 0.25) (layer "F.Cu") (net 23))
 (segment (start 106.5 59.5) (end 107.5 59.5) (width 0.25) (layer "F.Cu") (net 23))
 (segment (start 104 61.5) (end 104 62.5) (width 0.25) (layer "F.Cu") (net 23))
 (segment (start 104 62.5) (end 103.714 62.786) (width 0.25) (layer "F.Cu") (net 23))
 (segment (start 101.435 60.246) (end 103.746 60.246) (width 0.25) (layer "F.Cu") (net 23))
 (segment (start 104.5 61.5) (end 106.5 59.5) (width 0.25) (layer "F.Cu") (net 23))
 (segment (start 168 50.5) (end 113.5 50.5) (width 0.25) (layer "F.Cu") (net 23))
 (segment (start 107.5 56.5) (end 107.5 59.5) (width 0.25) (layer "F.Cu") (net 23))
 (segment (start 104 61.5) (end 104.5 61.5) (width 0.25) (layer "F.Cu") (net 23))
 (segment (start 104 60.5) (end 104 61.5) (width 0.25) (layer "F.Cu") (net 23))
 (segment (start 168.778 52.88) (end 168.778 51.278) (width 0.25) (layer "F.Cu") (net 23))
 (segment (start 113.5 50.5) (end 107.5 56.5) (width 0.25) (layer "F.Cu") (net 23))
 (segment (start 168.778 51.278) (end 168 50.5) (width 0.25) (layer "F.Cu") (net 23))
 (segment (start 105.715 64.056) (end 105.81 64.151) (width 0.25) (layer "F.Cu") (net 3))
 (segment (start 96.485 64.056) (end 97.929 65.5) (width 0.25) (layer "F.Cu") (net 3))
 (segment (start 101.435 64.056) (end 105.715 64.056) (width 0.25) (layer "F.Cu") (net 3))
 (segment (start 97.929 65.5) (end 99.991 65.5) (width 0.25) (layer "F.Cu") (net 3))
 (segment (start 99.991 65.5) (end 101.435 64.056) (width 0.25) (layer "F.Cu") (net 3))
 (segment (start 105.46 68.151) (end 105.81 67.801) (width 0.25) (layer "F.Cu") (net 3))
 (segment (start 105.81 67.801) (end 105.81 64.151) (width 0.25) (layer "F.Cu") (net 3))
 (segment (start 117.5 64.5) (end 117.499 64.501) (width 0.25) (layer "F.Cu") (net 9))
 (segment (start 117.5 63) (end 117.5 64.5) (width 0.25) (layer "F.Cu") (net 9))
 (segment (start 117.499 64.501) (end 113.79 64.501) (width 0.25) (layer "F.Cu") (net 9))
 (segment (start 144.5 57.5) (end 102 100) (width 0.25) (layer "F.Cu") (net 25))
 (segment (start 79.26 100.12) (end 79.26 105.5) (width 0.25) (layer "F.Cu") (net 25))
 (segment (start 79.38 100) (end 79.26 100.12) (width 0.25) (layer "F.Cu") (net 25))
 (segment (start 161.158 56.842) (end 160.5 57.5) (width 0.25) (layer "F.Cu") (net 25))
 (segment (start 161.158 52.88) (end 161.158 56.842) (width 0.25) (layer "F.Cu") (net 25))
 (segment (start 160.5 57.5) (end 144.5 57.5) (width 0.25) (layer "F.Cu") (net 25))
 (segment (start 102 100) (end 79.38 100) (width 0.25) (layer "F.Cu") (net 25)))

